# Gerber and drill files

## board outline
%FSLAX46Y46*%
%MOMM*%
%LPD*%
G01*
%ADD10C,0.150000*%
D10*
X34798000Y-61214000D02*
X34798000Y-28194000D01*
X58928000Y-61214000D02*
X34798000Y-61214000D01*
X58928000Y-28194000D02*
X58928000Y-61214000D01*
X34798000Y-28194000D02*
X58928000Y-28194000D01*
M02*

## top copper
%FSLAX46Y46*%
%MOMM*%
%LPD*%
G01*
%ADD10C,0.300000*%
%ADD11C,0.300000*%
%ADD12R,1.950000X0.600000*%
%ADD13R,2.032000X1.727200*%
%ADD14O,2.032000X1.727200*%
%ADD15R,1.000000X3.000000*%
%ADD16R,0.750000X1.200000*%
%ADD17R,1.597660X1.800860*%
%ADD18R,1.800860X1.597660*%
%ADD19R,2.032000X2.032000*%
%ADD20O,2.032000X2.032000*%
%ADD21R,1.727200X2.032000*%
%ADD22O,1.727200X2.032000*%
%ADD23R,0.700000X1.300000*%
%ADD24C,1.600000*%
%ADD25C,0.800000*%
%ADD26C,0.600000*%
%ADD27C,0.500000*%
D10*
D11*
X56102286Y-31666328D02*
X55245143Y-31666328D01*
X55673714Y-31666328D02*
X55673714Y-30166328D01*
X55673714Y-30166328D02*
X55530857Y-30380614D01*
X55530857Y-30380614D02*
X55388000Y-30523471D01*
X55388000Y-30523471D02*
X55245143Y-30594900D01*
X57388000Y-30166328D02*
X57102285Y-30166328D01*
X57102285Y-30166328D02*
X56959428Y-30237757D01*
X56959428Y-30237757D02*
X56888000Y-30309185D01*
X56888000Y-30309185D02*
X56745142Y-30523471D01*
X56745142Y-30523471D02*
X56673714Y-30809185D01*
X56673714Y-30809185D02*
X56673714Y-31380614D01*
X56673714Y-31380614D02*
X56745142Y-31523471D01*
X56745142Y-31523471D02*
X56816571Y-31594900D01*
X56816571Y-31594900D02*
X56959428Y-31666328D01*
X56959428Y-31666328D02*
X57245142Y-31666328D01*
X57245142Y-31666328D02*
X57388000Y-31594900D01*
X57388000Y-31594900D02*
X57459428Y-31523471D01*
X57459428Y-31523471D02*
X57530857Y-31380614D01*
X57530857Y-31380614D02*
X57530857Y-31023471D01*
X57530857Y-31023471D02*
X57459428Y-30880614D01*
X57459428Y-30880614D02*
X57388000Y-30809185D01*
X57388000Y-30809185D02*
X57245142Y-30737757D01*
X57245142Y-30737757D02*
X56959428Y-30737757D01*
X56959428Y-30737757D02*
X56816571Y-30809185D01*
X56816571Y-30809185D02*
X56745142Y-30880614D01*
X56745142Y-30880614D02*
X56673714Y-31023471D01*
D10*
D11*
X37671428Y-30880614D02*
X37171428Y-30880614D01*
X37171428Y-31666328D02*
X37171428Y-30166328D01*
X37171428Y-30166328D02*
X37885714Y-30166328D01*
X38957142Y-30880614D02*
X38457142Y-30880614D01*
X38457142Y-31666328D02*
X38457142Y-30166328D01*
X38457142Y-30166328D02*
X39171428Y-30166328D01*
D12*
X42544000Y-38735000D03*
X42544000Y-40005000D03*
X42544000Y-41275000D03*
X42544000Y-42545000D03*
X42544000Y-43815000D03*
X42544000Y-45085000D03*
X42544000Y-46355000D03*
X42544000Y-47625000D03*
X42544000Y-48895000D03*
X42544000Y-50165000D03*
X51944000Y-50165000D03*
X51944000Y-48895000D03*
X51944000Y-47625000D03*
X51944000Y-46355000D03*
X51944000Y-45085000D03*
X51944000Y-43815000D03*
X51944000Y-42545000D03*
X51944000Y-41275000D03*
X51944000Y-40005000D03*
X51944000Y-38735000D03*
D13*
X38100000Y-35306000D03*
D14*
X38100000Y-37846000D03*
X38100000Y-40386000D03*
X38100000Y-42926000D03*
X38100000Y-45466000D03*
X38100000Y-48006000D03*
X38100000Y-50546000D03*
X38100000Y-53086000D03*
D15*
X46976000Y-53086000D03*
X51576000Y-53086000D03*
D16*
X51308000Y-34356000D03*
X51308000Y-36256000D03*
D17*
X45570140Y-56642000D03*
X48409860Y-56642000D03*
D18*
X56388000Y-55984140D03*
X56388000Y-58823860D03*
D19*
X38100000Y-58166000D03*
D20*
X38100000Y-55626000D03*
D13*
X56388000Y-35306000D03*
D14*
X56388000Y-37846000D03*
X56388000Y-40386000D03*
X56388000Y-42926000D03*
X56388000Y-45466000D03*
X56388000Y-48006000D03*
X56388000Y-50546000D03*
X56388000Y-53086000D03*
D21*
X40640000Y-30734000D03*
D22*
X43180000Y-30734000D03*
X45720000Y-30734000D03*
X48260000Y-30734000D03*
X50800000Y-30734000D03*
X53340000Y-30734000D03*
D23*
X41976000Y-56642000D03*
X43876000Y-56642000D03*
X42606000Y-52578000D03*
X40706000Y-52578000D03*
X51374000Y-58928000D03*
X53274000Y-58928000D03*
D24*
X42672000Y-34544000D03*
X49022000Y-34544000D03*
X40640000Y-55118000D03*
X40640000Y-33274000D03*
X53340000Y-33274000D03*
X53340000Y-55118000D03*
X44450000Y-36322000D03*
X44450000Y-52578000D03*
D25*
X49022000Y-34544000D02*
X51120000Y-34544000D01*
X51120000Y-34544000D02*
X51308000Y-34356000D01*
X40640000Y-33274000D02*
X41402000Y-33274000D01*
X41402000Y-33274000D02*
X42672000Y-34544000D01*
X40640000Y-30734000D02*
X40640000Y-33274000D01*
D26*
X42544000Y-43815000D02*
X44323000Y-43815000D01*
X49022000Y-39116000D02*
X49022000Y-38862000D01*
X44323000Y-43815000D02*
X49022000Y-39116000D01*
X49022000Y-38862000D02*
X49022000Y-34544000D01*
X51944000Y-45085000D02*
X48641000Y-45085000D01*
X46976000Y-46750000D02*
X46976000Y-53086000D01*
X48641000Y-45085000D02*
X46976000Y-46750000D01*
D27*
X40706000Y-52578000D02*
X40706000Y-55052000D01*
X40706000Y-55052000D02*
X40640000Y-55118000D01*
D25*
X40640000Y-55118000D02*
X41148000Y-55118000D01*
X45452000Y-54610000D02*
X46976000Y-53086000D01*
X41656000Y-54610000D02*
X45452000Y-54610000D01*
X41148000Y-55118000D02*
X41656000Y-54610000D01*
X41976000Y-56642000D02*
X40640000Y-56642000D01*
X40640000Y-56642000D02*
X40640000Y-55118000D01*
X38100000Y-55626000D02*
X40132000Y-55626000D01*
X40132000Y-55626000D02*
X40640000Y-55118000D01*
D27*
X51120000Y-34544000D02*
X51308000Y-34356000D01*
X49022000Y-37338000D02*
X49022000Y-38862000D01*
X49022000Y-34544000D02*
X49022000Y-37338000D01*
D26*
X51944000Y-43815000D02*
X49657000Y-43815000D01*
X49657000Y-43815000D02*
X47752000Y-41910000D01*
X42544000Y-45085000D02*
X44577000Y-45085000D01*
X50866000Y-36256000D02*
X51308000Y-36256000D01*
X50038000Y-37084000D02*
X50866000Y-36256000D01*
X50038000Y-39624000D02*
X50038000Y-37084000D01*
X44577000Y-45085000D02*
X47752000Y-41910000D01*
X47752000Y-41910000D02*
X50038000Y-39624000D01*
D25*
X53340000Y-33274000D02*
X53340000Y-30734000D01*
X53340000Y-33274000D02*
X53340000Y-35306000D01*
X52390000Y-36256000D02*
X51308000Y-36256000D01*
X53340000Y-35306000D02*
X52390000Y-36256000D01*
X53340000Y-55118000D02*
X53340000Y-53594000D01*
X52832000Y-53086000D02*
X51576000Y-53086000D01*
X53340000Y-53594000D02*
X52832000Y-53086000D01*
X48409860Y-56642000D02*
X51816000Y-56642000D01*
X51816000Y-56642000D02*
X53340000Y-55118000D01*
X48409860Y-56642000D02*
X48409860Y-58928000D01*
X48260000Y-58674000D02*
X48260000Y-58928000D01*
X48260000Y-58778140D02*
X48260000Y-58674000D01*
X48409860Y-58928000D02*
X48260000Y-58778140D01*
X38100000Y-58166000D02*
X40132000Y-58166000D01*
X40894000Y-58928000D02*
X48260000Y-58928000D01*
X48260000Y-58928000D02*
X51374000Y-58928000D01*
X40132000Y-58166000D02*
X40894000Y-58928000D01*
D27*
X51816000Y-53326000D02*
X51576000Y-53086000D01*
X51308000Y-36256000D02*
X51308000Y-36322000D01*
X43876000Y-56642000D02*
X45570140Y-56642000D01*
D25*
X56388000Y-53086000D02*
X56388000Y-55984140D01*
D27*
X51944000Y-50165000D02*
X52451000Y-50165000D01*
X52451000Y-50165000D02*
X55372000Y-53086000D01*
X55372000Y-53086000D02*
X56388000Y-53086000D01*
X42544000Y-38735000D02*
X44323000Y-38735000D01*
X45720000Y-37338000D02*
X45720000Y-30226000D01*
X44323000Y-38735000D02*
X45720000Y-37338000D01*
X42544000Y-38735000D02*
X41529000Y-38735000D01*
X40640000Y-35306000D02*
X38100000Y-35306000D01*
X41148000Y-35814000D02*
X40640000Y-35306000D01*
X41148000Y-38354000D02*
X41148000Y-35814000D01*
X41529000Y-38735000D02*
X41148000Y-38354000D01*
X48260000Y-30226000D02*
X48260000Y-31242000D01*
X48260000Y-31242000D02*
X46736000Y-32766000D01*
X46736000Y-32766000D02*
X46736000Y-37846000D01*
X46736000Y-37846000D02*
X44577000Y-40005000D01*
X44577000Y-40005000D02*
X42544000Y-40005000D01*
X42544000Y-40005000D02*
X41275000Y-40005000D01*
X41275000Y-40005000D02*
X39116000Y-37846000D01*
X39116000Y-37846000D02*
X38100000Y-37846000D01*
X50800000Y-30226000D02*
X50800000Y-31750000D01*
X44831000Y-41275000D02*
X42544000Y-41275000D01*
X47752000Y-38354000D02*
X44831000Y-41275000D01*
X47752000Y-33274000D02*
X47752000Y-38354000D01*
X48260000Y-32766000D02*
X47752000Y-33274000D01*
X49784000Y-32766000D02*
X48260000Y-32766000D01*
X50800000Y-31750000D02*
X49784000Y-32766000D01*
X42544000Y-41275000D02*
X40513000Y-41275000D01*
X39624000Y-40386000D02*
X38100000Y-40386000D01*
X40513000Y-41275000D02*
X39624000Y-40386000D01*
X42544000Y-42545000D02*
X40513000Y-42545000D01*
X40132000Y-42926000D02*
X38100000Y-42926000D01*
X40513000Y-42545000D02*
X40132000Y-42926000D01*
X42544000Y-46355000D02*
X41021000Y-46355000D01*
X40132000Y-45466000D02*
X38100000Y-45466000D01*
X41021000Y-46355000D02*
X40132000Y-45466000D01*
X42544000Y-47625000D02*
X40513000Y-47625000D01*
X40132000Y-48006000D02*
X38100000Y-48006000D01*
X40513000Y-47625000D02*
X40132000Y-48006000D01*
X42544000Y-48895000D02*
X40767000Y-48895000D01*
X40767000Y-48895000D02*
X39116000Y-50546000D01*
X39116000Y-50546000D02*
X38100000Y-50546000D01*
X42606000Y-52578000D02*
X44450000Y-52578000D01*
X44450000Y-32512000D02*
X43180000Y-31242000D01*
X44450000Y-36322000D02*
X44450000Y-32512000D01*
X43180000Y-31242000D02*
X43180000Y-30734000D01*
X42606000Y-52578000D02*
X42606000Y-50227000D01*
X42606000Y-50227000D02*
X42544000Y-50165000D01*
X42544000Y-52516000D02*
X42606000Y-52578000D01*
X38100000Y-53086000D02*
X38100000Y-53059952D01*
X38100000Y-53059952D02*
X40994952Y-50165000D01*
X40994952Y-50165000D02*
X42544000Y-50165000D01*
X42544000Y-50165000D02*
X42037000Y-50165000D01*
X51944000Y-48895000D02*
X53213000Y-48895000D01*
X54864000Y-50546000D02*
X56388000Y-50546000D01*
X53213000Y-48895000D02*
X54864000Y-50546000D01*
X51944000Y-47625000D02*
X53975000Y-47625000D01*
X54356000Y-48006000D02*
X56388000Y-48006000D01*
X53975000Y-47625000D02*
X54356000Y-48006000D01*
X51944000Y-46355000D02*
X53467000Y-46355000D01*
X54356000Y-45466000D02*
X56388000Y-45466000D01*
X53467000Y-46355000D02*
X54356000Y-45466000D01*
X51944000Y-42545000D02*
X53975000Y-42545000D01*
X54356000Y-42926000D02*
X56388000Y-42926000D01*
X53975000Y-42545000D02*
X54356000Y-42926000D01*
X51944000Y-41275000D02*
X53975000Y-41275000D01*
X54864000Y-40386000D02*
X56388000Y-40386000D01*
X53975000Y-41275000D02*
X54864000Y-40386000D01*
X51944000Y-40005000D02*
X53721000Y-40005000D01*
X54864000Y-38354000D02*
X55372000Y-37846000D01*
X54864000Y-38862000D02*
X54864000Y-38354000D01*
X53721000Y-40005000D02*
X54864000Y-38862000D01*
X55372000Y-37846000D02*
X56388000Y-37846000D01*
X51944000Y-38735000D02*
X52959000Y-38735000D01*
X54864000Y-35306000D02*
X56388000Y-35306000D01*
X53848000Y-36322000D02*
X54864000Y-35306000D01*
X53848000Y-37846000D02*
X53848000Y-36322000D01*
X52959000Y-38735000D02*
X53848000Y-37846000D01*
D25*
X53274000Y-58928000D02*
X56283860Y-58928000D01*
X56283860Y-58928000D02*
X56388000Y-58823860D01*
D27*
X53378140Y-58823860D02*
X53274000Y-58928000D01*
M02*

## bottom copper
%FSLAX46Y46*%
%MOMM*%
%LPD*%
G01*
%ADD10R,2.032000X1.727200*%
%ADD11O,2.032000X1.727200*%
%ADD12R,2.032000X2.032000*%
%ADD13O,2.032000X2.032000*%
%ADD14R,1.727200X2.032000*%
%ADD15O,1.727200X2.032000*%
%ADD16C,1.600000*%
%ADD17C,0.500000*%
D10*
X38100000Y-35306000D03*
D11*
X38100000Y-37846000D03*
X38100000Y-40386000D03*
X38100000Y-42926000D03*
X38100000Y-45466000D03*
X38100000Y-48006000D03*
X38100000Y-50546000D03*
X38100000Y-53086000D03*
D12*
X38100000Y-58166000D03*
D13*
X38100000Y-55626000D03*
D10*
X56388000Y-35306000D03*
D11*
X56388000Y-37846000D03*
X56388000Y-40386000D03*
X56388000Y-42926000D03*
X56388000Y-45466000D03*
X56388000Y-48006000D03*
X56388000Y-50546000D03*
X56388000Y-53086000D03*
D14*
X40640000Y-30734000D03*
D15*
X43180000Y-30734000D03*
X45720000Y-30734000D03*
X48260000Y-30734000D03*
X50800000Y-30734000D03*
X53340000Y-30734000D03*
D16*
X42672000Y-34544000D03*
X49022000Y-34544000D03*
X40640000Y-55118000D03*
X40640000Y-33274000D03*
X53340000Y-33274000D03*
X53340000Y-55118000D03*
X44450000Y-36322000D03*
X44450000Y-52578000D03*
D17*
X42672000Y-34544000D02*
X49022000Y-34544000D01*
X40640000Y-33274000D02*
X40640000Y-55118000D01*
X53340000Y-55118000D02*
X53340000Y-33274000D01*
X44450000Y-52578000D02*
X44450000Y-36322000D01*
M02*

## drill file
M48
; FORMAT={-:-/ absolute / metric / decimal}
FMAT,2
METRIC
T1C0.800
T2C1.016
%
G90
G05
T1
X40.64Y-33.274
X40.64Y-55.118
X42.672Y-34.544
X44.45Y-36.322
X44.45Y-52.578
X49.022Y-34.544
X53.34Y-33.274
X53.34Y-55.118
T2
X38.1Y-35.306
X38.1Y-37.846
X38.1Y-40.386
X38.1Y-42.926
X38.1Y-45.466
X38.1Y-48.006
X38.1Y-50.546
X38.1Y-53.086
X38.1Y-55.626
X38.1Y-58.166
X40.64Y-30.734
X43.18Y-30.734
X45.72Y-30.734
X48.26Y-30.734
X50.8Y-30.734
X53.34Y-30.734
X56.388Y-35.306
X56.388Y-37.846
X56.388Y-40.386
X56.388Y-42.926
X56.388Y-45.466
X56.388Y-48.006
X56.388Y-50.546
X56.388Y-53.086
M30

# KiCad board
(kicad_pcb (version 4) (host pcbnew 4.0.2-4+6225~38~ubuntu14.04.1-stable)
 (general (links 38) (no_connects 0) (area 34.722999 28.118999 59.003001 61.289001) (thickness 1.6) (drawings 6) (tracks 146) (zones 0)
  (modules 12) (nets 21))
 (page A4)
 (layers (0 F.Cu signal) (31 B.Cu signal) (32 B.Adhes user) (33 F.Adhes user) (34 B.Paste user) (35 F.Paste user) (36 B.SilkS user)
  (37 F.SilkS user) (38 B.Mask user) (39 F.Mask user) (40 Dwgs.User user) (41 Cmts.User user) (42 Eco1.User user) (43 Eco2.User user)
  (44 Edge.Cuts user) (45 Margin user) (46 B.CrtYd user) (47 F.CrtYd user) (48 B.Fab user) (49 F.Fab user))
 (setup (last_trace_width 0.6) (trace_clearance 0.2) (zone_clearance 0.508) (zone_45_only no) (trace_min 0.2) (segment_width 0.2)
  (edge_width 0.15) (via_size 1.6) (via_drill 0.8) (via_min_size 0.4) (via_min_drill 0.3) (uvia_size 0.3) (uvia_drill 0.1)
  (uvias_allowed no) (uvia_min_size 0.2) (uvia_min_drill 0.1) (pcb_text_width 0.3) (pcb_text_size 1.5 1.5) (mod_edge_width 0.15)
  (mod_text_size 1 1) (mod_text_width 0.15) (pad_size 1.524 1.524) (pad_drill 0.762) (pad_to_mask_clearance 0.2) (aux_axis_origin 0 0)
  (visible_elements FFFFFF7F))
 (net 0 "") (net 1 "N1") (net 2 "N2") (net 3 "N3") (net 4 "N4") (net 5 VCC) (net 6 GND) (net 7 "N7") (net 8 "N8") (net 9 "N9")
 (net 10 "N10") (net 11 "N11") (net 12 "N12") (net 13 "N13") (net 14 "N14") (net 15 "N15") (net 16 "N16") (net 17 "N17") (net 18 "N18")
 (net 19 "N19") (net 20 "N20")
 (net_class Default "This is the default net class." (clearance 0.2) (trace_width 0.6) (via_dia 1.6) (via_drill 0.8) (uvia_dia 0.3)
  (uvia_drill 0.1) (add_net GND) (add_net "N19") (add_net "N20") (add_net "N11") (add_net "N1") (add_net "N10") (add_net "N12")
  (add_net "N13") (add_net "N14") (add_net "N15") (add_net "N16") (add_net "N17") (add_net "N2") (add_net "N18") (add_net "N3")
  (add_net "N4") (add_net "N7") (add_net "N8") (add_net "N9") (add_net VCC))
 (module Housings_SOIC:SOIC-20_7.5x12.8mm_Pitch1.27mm (layer F.Cu) (at 47.244 44.45)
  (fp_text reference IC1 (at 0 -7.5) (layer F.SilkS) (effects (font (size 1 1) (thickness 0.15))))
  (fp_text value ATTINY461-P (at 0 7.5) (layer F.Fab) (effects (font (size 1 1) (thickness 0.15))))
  (pad 1 smd rect (at -4.7 -5.715) (size 1.95 0.6) (layers F.Cu F.Paste F.Mask) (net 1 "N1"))
  (pad 2 smd rect (at -4.7 -4.445) (size 1.95 0.6) (layers F.Cu F.Paste F.Mask) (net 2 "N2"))
  (pad 3 smd rect (at -4.7 -3.175) (size 1.95 0.6) (layers F.Cu F.Paste F.Mask) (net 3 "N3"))
  (pad 4 smd rect (at -4.7 -1.905) (size 1.95 0.6) (layers F.Cu F.Paste F.Mask) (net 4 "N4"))
  (pad 5 smd rect (at -4.7 -0.635) (size 1.95 0.6) (layers F.Cu F.Paste F.Mask) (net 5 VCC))
  (pad 6 smd rect (at -4.7 0.635) (size 1.95 0.6) (layers F.Cu F.Paste F.Mask) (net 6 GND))
  (pad 7 smd rect (at -4.7 1.905) (size 1.95 0.6) (layers F.Cu F.Paste F.Mask) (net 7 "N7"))
  (pad 8 smd rect (at -4.7 3.175) (size 1.95 0.6) (layers F.Cu F.Paste F.Mask) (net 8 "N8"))
  (pad 9 smd rect (at -4.7 4.445) (size 1.95 0.6) (layers F.Cu F.Paste F.Mask) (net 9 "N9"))
  (pad 10 smd rect (at -4.7 5.715) (size 1.95 0.6) (layers F.Cu F.Paste F.Mask) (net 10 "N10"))
  (pad 11 smd rect (at 4.7 5.715) (size 1.95 0.6) (layers F.Cu F.Paste F.Mask) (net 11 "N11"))
  (pad 12 smd rect (at 4.7 4.445) (size 1.95 0.6) (layers F.Cu F.Paste F.Mask) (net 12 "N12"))
  (pad 13 smd rect (at 4.7 3.175) (size 1.95 0.6) (layers F.Cu F.Paste F.Mask) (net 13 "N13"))
  (pad 14 smd rect (at 4.7 1.905) (size 1.95 0.6) (layers F.Cu F.Paste F.Mask) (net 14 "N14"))
  (pad 15 smd rect (at 4.7 0.635) (size 1.95 0.6) (layers F.Cu F.Paste F.Mask) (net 5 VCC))
  (pad 16 smd rect (at 4.7 -0.635) (size 1.95 0.6) (layers F.Cu F.Paste F.Mask) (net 6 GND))
  (pad 17 smd rect (at 4.7 -1.905) (size 1.95 0.6) (layers F.Cu F.Paste F.Mask) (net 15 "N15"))
  (pad 18 smd rect (at 4.7 -3.175) (size 1.95 0.6) (layers F.Cu F.Paste F.Mask) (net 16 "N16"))
  (pad 19 smd rect (at 4.7 -4.445) (size 1.95 0.6) (layers F.Cu F.Paste F.Mask) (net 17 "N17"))
  (pad 20 smd rect (at 4.7 -5.715) (size 1.95 0.6) (layers F.Cu F.Paste F.Mask) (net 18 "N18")))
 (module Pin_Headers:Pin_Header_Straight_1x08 (layer F.Cu) (at 38.1 35.306)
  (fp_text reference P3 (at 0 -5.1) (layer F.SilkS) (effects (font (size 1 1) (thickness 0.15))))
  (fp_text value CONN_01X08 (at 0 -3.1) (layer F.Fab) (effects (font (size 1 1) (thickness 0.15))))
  (pad 1 thru_hole rect (at 0 0) (size 2.032 1.7272) (drill 1.016) (layers *.Cu *.Mask F.SilkS) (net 1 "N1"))
  (pad 2 thru_hole oval (at 0 2.54) (size 2.032 1.7272) (drill 1.016) (layers *.Cu *.Mask F.SilkS) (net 2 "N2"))
  (pad 3 thru_hole oval (at 0 5.08) (size 2.032 1.7272) (drill 1.016) (layers *.Cu *.Mask F.SilkS) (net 3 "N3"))
  (pad 4 thru_hole oval (at 0 7.62) (size 2.032 1.7272) (drill 1.016) (layers *.Cu *.Mask F.SilkS) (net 4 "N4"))
  (pad 5 thru_hole oval (at 0 10.16) (size 2.032 1.7272) (drill 1.016) (layers *.Cu *.Mask F.SilkS) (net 7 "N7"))
  (pad 6 thru_hole oval (at 0 12.7) (size 2.032 1.7272) (drill 1.016) (layers *.Cu *.Mask F.SilkS) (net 8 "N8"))
  (pad 7 thru_hole oval (at 0 15.24) (size 2.032 1.7272) (drill 1.016) (layers *.Cu *.Mask F.SilkS) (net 9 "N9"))
  (pad 8 thru_hole oval (at 0 17.78) (size 2.032 1.7272) (drill 1.016) (layers *.Cu *.Mask F.SilkS) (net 10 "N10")))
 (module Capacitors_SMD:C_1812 (layer F.Cu) (at 49.276 53.086)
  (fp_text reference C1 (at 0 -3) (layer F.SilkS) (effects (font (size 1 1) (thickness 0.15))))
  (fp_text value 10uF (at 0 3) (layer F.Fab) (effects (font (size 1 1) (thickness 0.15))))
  (pad 1 smd rect (at -2.3 0) (size 1 3) (layers F.Cu F.Paste F.Mask) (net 5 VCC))
  (pad 2 smd rect (at 2.3 0) (size 1 3) (layers F.Cu F.Paste F.Mask) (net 6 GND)))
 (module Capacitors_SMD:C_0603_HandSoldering (layer F.Cu) (at 51.308 35.306 270)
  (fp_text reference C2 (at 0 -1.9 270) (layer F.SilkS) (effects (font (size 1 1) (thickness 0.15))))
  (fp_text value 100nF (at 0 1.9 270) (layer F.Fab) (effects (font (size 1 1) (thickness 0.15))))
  (pad 1 smd rect (at -0.95 0 270) (size 1.2 0.75) (layers F.Cu F.Paste F.Mask) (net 5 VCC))
  (pad 2 smd rect (at 0.95 0 270) (size 1.2 0.75) (layers F.Cu F.Paste F.Mask) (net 6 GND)))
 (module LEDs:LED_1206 (layer F.Cu) (at 46.99 56.642 180)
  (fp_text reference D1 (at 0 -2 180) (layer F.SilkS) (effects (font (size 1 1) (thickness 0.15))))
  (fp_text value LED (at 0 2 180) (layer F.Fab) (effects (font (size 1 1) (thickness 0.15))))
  (pad 2 smd rect (at 1.41986 0) (size 1.59766 1.80086) (layers F.Cu F.Paste F.Mask) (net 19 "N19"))
  (pad 1 smd rect (at -1.41986 0) (size 1.59766 1.80086) (layers F.Cu F.Paste F.Mask) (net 6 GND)))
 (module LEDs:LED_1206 (layer F.Cu) (at 56.388 57.404 90)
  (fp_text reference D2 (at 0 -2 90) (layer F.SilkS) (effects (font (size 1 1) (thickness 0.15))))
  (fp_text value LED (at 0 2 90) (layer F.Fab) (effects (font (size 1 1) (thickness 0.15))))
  (pad 2 smd rect (at 1.41986 0 270) (size 1.59766 1.80086) (layers F.Cu F.Paste F.Mask) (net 11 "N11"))
  (pad 1 smd rect (at -1.41986 0 270) (size 1.59766 1.80086) (layers F.Cu F.Paste F.Mask) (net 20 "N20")))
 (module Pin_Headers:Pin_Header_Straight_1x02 (layer F.Cu) (at 38.1 58.166 180)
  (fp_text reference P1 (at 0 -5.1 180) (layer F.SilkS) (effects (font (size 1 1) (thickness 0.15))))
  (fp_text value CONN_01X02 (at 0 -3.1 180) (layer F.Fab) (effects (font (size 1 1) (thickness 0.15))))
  (pad 1 thru_hole rect (at 0 0 180) (size 2.032 2.032) (drill 1.016) (layers *.Cu *.Mask F.SilkS) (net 6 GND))
  (pad 2 thru_hole oval (at 0 2.54 180) (size 2.032 2.032) (drill 1.016) (layers *.Cu *.Mask F.SilkS) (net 5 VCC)))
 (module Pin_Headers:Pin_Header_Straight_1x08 (layer F.Cu) (at 56.388 35.306)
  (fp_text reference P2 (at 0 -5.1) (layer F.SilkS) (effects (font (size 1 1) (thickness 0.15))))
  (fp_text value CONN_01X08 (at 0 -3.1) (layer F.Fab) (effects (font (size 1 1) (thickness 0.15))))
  (pad 1 thru_hole rect (at 0 0) (size 2.032 1.7272) (drill 1.016) (layers *.Cu *.Mask F.SilkS) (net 18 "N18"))
  (pad 2 thru_hole oval (at 0 2.54) (size 2.032 1.7272) (drill 1.016) (layers *.Cu *.Mask F.SilkS) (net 17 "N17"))
  (pad 3 thru_hole oval (at 0 5.08) (size 2.032 1.7272) (drill 1.016) (layers *.Cu *.Mask F.SilkS) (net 16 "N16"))
  (pad 4 thru_hole oval (at 0 7.62) (size 2.032 1.7272) (drill 1.016) (layers *.Cu *.Mask F.SilkS) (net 15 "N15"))
  (pad 5 thru_hole oval (at 0 10.16) (size 2.032 1.7272) (drill 1.016) (layers *.Cu *.Mask F.SilkS) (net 14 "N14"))
  (pad 6 thru_hole oval (at 0 12.7) (size 2.032 1.7272) (drill 1.016) (layers *.Cu *.Mask F.SilkS) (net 13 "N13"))
  (pad 7 thru_hole oval (at 0 15.24) (size 2.032 1.7272) (drill 1.016) (layers *.Cu *.Mask F.SilkS) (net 12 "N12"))
  (pad 8 thru_hole oval (at 0 17.78) (size 2.032 1.7272) (drill 1.016) (layers *.Cu *.Mask F.SilkS) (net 11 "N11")))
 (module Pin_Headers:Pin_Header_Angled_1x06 (layer F.Cu) (at 40.64 30.734 90)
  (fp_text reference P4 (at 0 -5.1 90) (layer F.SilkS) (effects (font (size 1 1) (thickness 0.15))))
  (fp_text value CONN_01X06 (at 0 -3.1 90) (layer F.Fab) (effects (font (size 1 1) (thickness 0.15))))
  (pad 1 thru_hole rect (at 0 0 90) (size 2.032 1.7272) (drill 1.016) (layers *.Cu *.Mask F.SilkS) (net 5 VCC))
  (pad 2 thru_hole oval (at 0 2.54 90) (size 2.032 1.7272) (drill 1.016) (layers *.Cu *.Mask F.SilkS) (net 10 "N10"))
  (pad 3 thru_hole oval (at 0 5.08 90) (size 2.032 1.7272) (drill 1.016) (layers *.Cu *.Mask F.SilkS) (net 1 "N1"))
  (pad 4 thru_hole oval (at 0 7.62 90) (size 2.032 1.7272) (drill 1.016) (layers *.Cu *.Mask F.SilkS) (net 2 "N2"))
  (pad 5 thru_hole oval (at 0 10.16 90) (size 2.032 1.7272) (drill 1.016) (layers *.Cu *.Mask F.SilkS) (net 3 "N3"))
  (pad 6 thru_hole oval (at 0 12.7 90) (size 2.032 1.7272) (drill 1.016) (layers *.Cu *.Mask F.SilkS) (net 6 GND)))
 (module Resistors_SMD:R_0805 (layer F.Cu) (at 42.926 56.642)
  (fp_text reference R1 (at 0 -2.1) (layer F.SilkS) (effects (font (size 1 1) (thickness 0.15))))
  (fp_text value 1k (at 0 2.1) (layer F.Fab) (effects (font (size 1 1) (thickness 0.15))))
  (pad 1 smd rect (at -0.95 0) (size 0.7 1.3) (layers F.Cu F.Paste F.Mask) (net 5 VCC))
  (pad 2 smd rect (at 0.95 0) (size 0.7 1.3) (layers F.Cu F.Paste F.Mask) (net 19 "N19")))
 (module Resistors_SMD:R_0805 (layer F.Cu) (at 41.656 52.578 180)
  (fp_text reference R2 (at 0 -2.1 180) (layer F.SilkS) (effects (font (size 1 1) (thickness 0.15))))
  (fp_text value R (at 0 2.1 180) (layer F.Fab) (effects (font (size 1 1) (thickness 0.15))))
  (pad 1 smd rect (at -0.95 0 180) (size 0.7 1.3) (layers F.Cu F.Paste F.Mask) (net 10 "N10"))
  (pad 2 smd rect (at 0.95 0 180) (size 0.7 1.3) (layers F.Cu F.Paste F.Mask) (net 5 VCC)))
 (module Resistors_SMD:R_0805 (layer F.Cu) (at 52.324 58.928)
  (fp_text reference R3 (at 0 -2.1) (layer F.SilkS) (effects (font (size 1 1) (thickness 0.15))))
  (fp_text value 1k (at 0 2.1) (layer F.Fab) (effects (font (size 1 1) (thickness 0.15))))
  (pad 1 smd rect (at -0.95 0) (size 0.7 1.3) (layers F.Cu F.Paste F.Mask) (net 6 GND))
  (pad 2 smd rect (at 0.95 0) (size 0.7 1.3) (layers F.Cu F.Paste F.Mask) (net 20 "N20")))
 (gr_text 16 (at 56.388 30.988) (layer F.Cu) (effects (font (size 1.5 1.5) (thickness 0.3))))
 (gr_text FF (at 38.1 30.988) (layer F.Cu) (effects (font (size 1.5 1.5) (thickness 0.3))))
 (gr_line (start 34.798 61.214) (end 34.798 28.194) (angle 90) (layer Edge.Cuts) (width 0.15))
 (gr_line (start 58.928 61.214) (end 34.798 61.214) (angle 90) (layer Edge.Cuts) (width 0.15))
 (gr_line (start 58.928 28.194) (end 58.928 61.214) (angle 90) (layer Edge.Cuts) (width 0.15))
 (gr_line (start 34.798 28.194) (end 58.928 28.194) (angle 90) (layer Edge.Cuts) (width 0.15))
 (segment (start 49.022 34.544) (end 51.12 34.544) (width 0.8) (layer F.Cu) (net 5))
 (segment (start 51.12 34.544) (end 51.308 34.356) (width 0.8) (layer F.Cu) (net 5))
 (segment (start 40.64 33.274) (end 41.402 33.274) (width 0.8) (layer F.Cu) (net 5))
 (via (at 42.672 34.544) (size 1.6) (drill 0.8) (layers F.Cu B.Cu) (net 5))
 (segment (start 42.672 34.544) (end 49.022 34.544) (width 0.5) (layer B.Cu) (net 5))
 (via (at 49.022 34.544) (size 1.6) (drill 0.8) (layers F.Cu B.Cu) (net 5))
 (segment (start 41.402 33.274) (end 42.672 34.544) (width 0.8) (layer F.Cu) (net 5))
 (segment (start 40.64 30.734) (end 40.64 33.274) (width 0.8) (layer F.Cu) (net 5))
 (via (at 40.64 55.118) (size 1.6) (drill 0.8) (layers F.Cu B.Cu) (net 5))
 (segment (start 40.64 33.274) (end 40.64 55.118) (width 0.5) (layer B.Cu) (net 5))
 (via (at 40.64 33.274) (size 1.6) (drill 0.8) (layers F.Cu B.Cu) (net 5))
 (segment (start 42.544 43.815) (end 44.323 43.815) (width 0.6) (layer F.Cu) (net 5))
 (segment (start 49.022 39.116) (end 49.022 38.862) (width 0.6) (layer F.Cu) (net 5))
 (segment (start 44.323 43.815) (end 49.022 39.116) (width 0.6) (layer F.Cu) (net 5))
 (segment (start 49.022 38.862) (end 49.022 34.544) (width 0.6) (layer F.Cu) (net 5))
 (segment (start 51.944 45.085) (end 48.641 45.085) (width 0.6) (layer F.Cu) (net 5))
 (segment (start 46.976 46.75) (end 46.976 53.086) (width 0.6) (layer F.Cu) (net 5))
 (segment (start 48.641 45.085) (end 46.976 46.75) (width 0.6) (layer F.Cu) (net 5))
 (segment (start 40.706 52.578) (end 40.706 55.052) (width 0.5) (layer F.Cu) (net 5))
 (segment (start 40.706 55.052) (end 40.64 55.118) (width 0.5) (layer F.Cu) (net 5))
 (segment (start 40.64 55.118) (end 41.148 55.118) (width 0.8) (layer F.Cu) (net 5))
 (segment (start 45.452 54.61) (end 46.976 53.086) (width 0.8) (layer F.Cu) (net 5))
 (segment (start 41.656 54.61) (end 45.452 54.61) (width 0.8) (layer F.Cu) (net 5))
 (segment (start 41.148 55.118) (end 41.656 54.61) (width 0.8) (layer F.Cu) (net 5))
 (segment (start 41.976 56.642) (end 40.64 56.642) (width 0.8) (layer F.Cu) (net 5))
 (segment (start 40.64 56.642) (end 40.64 55.118) (width 0.8) (layer F.Cu) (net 5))
 (segment (start 38.1 55.626) (end 40.132 55.626) (width 0.8) (layer F.Cu) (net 5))
 (segment (start 40.132 55.626) (end 40.64 55.118) (width 0.8) (layer F.Cu) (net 5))
 (segment (start 51.12 34.544) (end 51.308 34.356) (width 0.5) (layer F.Cu) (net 5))
 (segment (start 49.022 37.338) (end 49.022 38.862) (width 0.5) (layer F.Cu) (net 5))
 (segment (start 49.022 34.544) (end 49.022 37.338) (width 0.5) (layer F.Cu) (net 5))
 (segment (start 51.944 43.815) (end 49.657 43.815) (width 0.6) (layer F.Cu) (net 6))
 (segment (start 49.657 43.815) (end 47.752 41.91) (width 0.6) (layer F.Cu) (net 6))
 (segment (start 42.544 45.085) (end 44.577 45.085) (width 0.6) (layer F.Cu) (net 6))
 (segment (start 50.866 36.256) (end 51.308 36.256) (width 0.6) (layer F.Cu) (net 6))
 (segment (start 50.038 37.084) (end 50.866 36.256) (width 0.6) (layer F.Cu) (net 6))
 (segment (start 50.038 39.624) (end 50.038 37.084) (width 0.6) (layer F.Cu) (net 6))
 (segment (start 44.577 45.085) (end 47.752 41.91) (width 0.6) (layer F.Cu) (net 6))
 (segment (start 47.752 41.91) (end 50.038 39.624) (width 0.6) (layer F.Cu) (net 6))
 (segment (start 53.34 33.274) (end 53.34 30.734) (width 0.8) (layer F.Cu) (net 6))
 (segment (start 53.34 33.274) (end 53.34 35.306) (width 0.8) (layer F.Cu) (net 6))
 (segment (start 53.34 55.118) (end 53.34 33.274) (width 0.5) (layer B.Cu) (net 6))
 (via (at 53.34 33.274) (size 1.6) (drill 0.8) (layers F.Cu B.Cu) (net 6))
 (via (at 53.34 55.118) (size 1.6) (drill 0.8) (layers F.Cu B.Cu) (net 6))
 (segment (start 52.39 36.256) (end 51.308 36.256) (width 0.8) (layer F.Cu) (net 6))
 (segment (start 53.34 35.306) (end 52.39 36.256) (width 0.8) (layer F.Cu) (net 6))
 (segment (start 53.34 55.118) (end 53.34 53.594) (width 0.8) (layer F.Cu) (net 6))
 (segment (start 52.832 53.086) (end 51.576 53.086) (width 0.8) (layer F.Cu) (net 6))
 (segment (start 53.34 53.594) (end 52.832 53.086) (width 0.8) (layer F.Cu) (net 6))
 (segment (start 48.40986 56.642) (end 51.816 56.642) (width 0.8) (layer F.Cu) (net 6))
 (segment (start 51.816 56.642) (end 53.34 55.118) (width 0.8) (layer F.Cu) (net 6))
 (segment (start 48.40986 56.642) (end 48.40986 58.928) (width 0.8) (layer F.Cu) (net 6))
 (segment (start 48.26 58.674) (end 48.26 58.928) (width 0.8) (layer F.Cu) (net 6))
 (segment (start 48.26 58.77814) (end 48.26 58.674) (width 0.8) (layer F.Cu) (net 6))
 (segment (start 48.40986 58.928) (end 48.26 58.77814) (width 0.8) (layer F.Cu) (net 6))
 (segment (start 38.1 58.166) (end 40.132 58.166) (width 0.8) (layer F.Cu) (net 6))
 (segment (start 40.894 58.928) (end 48.26 58.928) (width 0.8) (layer F.Cu) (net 6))
 (segment (start 48.26 58.928) (end 51.374 58.928) (width 0.8) (layer F.Cu) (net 6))
 (segment (start 40.132 58.166) (end 40.894 58.928) (width 0.8) (layer F.Cu) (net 6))
 (segment (start 51.816 53.326) (end 51.576 53.086) (width 0.5) (layer F.Cu) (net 6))
 (segment (start 51.308 36.256) (end 51.308 36.322) (width 0.5) (layer F.Cu) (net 6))
 (segment (start 43.876 56.642) (end 45.57014 56.642) (width 0.5) (layer F.Cu) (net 19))
 (segment (start 56.388 53.086) (end 56.388 55.98414) (width 0.8) (layer F.Cu) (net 11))
 (segment (start 51.944 50.165) (end 52.451 50.165) (width 0.5) (layer F.Cu) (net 11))
 (segment (start 52.451 50.165) (end 55.372 53.086) (width 0.5) (layer F.Cu) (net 11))
 (segment (start 55.372 53.086) (end 56.388 53.086) (width 0.5) (layer F.Cu) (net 11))
 (segment (start 42.544 38.735) (end 44.323 38.735) (width 0.5) (layer F.Cu) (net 1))
 (segment (start 45.72 37.338) (end 45.72 30.226) (width 0.5) (layer F.Cu) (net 1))
 (segment (start 44.323 38.735) (end 45.72 37.338) (width 0.5) (layer F.Cu) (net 1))
 (segment (start 42.544 38.735) (end 41.529 38.735) (width 0.5) (layer F.Cu) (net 1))
 (segment (start 40.64 35.306) (end 38.1 35.306) (width 0.5) (layer F.Cu) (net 1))
 (segment (start 41.148 35.814) (end 40.64 35.306) (width 0.5) (layer F.Cu) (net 1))
 (segment (start 41.148 38.354) (end 41.148 35.814) (width 0.5) (layer F.Cu) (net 1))
 (segment (start 41.529 38.735) (end 41.148 38.354) (width 0.5) (layer F.Cu) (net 1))
 (segment (start 48.26 30.226) (end 48.26 31.242) (width 0.5) (layer F.Cu) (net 2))
 (segment (start 48.26 31.242) (end 46.736 32.766) (width 0.5) (layer F.Cu) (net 2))
 (segment (start 46.736 32.766) (end 46.736 37.846) (width 0.5) (layer F.Cu) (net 2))
 (segment (start 46.736 37.846) (end 44.577 40.005) (width 0.5) (layer F.Cu) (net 2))
 (segment (start 44.577 40.005) (end 42.544 40.005) (width 0.5) (layer F.Cu) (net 2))
 (segment (start 42.544 40.005) (end 41.275 40.005) (width 0.5) (layer F.Cu) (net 2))
 (segment (start 41.275 40.005) (end 39.116 37.846) (width 0.5) (layer F.Cu) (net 2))
 (segment (start 39.116 37.846) (end 38.1 37.846) (width 0.5) (layer F.Cu) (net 2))
 (segment (start 50.8 30.226) (end 50.8 31.75) (width 0.5) (layer F.Cu) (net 3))
 (segment (start 44.831 41.275) (end 42.544 41.275) (width 0.5) (layer F.Cu) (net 3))
 (segment (start 47.752 38.354) (end 44.831 41.275) (width 0.5) (layer F.Cu) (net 3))
 (segment (start 47.752 33.274) (end 47.752 38.354) (width 0.5) (layer F.Cu) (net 3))
 (segment (start 48.26 32.766) (end 47.752 33.274) (width 0.5) (layer F.Cu) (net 3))
 (segment (start 49.784 32.766) (end 48.26 32.766) (width 0.5) (layer F.Cu) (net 3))
 (segment (start 50.8 31.75) (end 49.784 32.766) (width 0.5) (layer F.Cu) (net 3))
 (segment (start 42.544 41.275) (end 40.513 41.275) (width 0.5) (layer F.Cu) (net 3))
 (segment (start 39.624 40.386) (end 38.1 40.386) (width 0.5) (layer F.Cu) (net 3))
 (segment (start 40.513 41.275) (end 39.624 40.386) (width 0.5) (layer F.Cu) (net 3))
 (segment (start 42.544 42.545) (end 40.513 42.545) (width 0.5) (layer F.Cu) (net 4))
 (segment (start 40.132 42.926) (end 38.1 42.926) (width 0.5) (layer F.Cu) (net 4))
 (segment (start 40.513 42.545) (end 40.132 42.926) (width 0.5) (layer F.Cu) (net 4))
 (segment (start 42.544 46.355) (end 41.021 46.355) (width 0.5) (layer F.Cu) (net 7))
 (segment (start 40.132 45.466) (end 38.1 45.466) (width 0.5) (layer F.Cu) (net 7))
 (segment (start 41.021 46.355) (end 40.132 45.466) (width 0.5) (layer F.Cu) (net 7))
 (segment (start 42.544 47.625) (end 40.513 47.625) (width 0.5) (layer F.Cu) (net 8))
 (segment (start 40.132 48.006) (end 38.1 48.006) (width 0.5) (layer F.Cu) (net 8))
 (segment (start 40.513 47.625) (end 40.132 48.006) (width 0.5) (layer F.Cu) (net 8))
 (segment (start 42.544 48.895) (end 40.767 48.895) (width 0.5) (layer F.Cu) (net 9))
 (segment (start 40.767 48.895) (end 39.116 50.546) (width 0.5) (layer F.Cu) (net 9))
 (segment (start 39.116 50.546) (end 38.1 50.546) (width 0.5) (layer F.Cu) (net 9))
 (segment (start 42.606 52.578) (end 44.45 52.578) (width 0.5) (layer F.Cu) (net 10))
 (segment (start 44.45 32.512) (end 43.18 31.242) (width 0.5) (layer F.Cu) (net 10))
 (segment (start 44.45 36.322) (end 44.45 32.512) (width 0.5) (layer F.Cu) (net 10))
 (via (at 44.45 36.322) (size 1.6) (drill 0.8) (layers F.Cu B.Cu) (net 10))
 (segment (start 44.45 52.578) (end 44.45 36.322) (width 0.5) (layer B.Cu) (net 10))
 (via (at 44.45 52.578) (size 1.6) (drill 0.8) (layers F.Cu B.Cu) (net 10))
 (segment (start 43.18 31.242) (end 43.18 30.734) (width 0.5) (layer F.Cu) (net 10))
 (segment (start 42.606 52.578) (end 42.606 50.227) (width 0.5) (layer F.Cu) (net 10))
 (segment (start 42.606 50.227) (end 42.544 50.165) (width 0.5) (layer F.Cu) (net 10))
 (segment (start 42.544 52.516) (end 42.606 52.578) (width 0.5) (layer F.Cu) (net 10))
 (segment (start 38.1 53.086) (end 38.1 53.059952) (width 0.5) (layer F.Cu) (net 10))
 (segment (start 38.1 53.059952) (end 40.994952 50.165) (width 0.5) (layer F.Cu) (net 10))
 (segment (start 40.994952 50.165) (end 42.544 50.165) (width 0.5) (layer F.Cu) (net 10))
 (segment (start 42.544 50.165) (end 42.037 50.165) (width 0.5) (layer F.Cu) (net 10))
 (segment (start 51.944 48.895) (end 53.213 48.895) (width 0.5) (layer F.Cu) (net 12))
 (segment (start 54.864 50.546) (end 56.388 50.546) (width 0.5) (layer F.Cu) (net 12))
 (segment (start 53.213 48.895) (end 54.864 50.546) (width 0.5) (layer F.Cu) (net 12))
 (segment (start 51.944 47.625) (end 53.975 47.625) (width 0.5) (layer F.Cu) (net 13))
 (segment (start 54.356 48.006) (end 56.388 48.006) (width 0.5) (layer F.Cu) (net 13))
 (segment (start 53.975 47.625) (end 54.356 48.006) (width 0.5) (layer F.Cu) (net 13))
 (segment (start 51.944 46.355) (end 53.467 46.355) (width 0.5) (layer F.Cu) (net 14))
 (segment (start 54.356 45.466) (end 56.388 45.466) (width 0.5) (layer F.Cu) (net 14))
 (segment (start 53.467 46.355) (end 54.356 45.466) (width 0.5) (layer F.Cu) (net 14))
 (segment (start 51.944 42.545) (end 53.975 42.545) (width 0.5) (layer F.Cu) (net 15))
 (segment (start 54.356 42.926) (end 56.388 42.926) (width 0.5) (layer F.Cu) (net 15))
 (segment (start 53.975 42.545) (end 54.356 42.926) (width 0.5) (layer F.Cu) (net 15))
 (segment (start 51.944 41.275) (end 53.975 41.275) (width 0.5) (layer F.Cu) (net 16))
 (segment (start 54.864 40.386) (end 56.388 40.386) (width 0.5) (layer F.Cu) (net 16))
 (segment (start 53.975 41.275) (end 54.864 40.386) (width 0.5) (layer F.Cu) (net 16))
 (segment (start 51.944 40.005) (end 53.721 40.005) (width 0.5) (layer F.Cu) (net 17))
 (segment (start 54.864 38.354) (end 55.372 37.846) (width 0.5) (layer F.Cu) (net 17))
 (segment (start 54.864 38.862) (end 54.864 38.354) (width 0.5) (layer F.Cu) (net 17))
 (segment (start 53.721 40.005) (end 54.864 38.862) (width 0.5) (layer F.Cu) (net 17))
 (segment (start 55.372 37.846) (end 56.388 37.846) (width 0.5) (layer F.Cu) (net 17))
 (segment (start 51.944 38.735) (end 52.959 38.735) (width 0.5) (layer F.Cu) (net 18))
 (segment (start 54.864 35.306) (end 56.388 35.306) (width 0.5) (layer F.Cu) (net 18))
 (segment (start 53.848 36.322) (end 54.864 35.306) (width 0.5) (layer F.Cu) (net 18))
 (segment (start 53.848 37.846) (end 53.848 36.322) (width 0.5) (layer F.Cu) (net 18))
 (segment (start 52.959 38.735) (end 53.848 37.846) (width 0.5) (layer F.Cu) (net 18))
 (segment (start 53.274 58.928) (end 56.28386 58.928) (width 0.8) (layer F.Cu) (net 20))
 (segment (start 56.28386 58.928) (end 56.388 58.82386) (width 0.8) (layer F.Cu) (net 20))
 (segment (start 53.37814 58.82386) (end 53.274 58.928) (width 0.5) (layer F.Cu) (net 20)))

